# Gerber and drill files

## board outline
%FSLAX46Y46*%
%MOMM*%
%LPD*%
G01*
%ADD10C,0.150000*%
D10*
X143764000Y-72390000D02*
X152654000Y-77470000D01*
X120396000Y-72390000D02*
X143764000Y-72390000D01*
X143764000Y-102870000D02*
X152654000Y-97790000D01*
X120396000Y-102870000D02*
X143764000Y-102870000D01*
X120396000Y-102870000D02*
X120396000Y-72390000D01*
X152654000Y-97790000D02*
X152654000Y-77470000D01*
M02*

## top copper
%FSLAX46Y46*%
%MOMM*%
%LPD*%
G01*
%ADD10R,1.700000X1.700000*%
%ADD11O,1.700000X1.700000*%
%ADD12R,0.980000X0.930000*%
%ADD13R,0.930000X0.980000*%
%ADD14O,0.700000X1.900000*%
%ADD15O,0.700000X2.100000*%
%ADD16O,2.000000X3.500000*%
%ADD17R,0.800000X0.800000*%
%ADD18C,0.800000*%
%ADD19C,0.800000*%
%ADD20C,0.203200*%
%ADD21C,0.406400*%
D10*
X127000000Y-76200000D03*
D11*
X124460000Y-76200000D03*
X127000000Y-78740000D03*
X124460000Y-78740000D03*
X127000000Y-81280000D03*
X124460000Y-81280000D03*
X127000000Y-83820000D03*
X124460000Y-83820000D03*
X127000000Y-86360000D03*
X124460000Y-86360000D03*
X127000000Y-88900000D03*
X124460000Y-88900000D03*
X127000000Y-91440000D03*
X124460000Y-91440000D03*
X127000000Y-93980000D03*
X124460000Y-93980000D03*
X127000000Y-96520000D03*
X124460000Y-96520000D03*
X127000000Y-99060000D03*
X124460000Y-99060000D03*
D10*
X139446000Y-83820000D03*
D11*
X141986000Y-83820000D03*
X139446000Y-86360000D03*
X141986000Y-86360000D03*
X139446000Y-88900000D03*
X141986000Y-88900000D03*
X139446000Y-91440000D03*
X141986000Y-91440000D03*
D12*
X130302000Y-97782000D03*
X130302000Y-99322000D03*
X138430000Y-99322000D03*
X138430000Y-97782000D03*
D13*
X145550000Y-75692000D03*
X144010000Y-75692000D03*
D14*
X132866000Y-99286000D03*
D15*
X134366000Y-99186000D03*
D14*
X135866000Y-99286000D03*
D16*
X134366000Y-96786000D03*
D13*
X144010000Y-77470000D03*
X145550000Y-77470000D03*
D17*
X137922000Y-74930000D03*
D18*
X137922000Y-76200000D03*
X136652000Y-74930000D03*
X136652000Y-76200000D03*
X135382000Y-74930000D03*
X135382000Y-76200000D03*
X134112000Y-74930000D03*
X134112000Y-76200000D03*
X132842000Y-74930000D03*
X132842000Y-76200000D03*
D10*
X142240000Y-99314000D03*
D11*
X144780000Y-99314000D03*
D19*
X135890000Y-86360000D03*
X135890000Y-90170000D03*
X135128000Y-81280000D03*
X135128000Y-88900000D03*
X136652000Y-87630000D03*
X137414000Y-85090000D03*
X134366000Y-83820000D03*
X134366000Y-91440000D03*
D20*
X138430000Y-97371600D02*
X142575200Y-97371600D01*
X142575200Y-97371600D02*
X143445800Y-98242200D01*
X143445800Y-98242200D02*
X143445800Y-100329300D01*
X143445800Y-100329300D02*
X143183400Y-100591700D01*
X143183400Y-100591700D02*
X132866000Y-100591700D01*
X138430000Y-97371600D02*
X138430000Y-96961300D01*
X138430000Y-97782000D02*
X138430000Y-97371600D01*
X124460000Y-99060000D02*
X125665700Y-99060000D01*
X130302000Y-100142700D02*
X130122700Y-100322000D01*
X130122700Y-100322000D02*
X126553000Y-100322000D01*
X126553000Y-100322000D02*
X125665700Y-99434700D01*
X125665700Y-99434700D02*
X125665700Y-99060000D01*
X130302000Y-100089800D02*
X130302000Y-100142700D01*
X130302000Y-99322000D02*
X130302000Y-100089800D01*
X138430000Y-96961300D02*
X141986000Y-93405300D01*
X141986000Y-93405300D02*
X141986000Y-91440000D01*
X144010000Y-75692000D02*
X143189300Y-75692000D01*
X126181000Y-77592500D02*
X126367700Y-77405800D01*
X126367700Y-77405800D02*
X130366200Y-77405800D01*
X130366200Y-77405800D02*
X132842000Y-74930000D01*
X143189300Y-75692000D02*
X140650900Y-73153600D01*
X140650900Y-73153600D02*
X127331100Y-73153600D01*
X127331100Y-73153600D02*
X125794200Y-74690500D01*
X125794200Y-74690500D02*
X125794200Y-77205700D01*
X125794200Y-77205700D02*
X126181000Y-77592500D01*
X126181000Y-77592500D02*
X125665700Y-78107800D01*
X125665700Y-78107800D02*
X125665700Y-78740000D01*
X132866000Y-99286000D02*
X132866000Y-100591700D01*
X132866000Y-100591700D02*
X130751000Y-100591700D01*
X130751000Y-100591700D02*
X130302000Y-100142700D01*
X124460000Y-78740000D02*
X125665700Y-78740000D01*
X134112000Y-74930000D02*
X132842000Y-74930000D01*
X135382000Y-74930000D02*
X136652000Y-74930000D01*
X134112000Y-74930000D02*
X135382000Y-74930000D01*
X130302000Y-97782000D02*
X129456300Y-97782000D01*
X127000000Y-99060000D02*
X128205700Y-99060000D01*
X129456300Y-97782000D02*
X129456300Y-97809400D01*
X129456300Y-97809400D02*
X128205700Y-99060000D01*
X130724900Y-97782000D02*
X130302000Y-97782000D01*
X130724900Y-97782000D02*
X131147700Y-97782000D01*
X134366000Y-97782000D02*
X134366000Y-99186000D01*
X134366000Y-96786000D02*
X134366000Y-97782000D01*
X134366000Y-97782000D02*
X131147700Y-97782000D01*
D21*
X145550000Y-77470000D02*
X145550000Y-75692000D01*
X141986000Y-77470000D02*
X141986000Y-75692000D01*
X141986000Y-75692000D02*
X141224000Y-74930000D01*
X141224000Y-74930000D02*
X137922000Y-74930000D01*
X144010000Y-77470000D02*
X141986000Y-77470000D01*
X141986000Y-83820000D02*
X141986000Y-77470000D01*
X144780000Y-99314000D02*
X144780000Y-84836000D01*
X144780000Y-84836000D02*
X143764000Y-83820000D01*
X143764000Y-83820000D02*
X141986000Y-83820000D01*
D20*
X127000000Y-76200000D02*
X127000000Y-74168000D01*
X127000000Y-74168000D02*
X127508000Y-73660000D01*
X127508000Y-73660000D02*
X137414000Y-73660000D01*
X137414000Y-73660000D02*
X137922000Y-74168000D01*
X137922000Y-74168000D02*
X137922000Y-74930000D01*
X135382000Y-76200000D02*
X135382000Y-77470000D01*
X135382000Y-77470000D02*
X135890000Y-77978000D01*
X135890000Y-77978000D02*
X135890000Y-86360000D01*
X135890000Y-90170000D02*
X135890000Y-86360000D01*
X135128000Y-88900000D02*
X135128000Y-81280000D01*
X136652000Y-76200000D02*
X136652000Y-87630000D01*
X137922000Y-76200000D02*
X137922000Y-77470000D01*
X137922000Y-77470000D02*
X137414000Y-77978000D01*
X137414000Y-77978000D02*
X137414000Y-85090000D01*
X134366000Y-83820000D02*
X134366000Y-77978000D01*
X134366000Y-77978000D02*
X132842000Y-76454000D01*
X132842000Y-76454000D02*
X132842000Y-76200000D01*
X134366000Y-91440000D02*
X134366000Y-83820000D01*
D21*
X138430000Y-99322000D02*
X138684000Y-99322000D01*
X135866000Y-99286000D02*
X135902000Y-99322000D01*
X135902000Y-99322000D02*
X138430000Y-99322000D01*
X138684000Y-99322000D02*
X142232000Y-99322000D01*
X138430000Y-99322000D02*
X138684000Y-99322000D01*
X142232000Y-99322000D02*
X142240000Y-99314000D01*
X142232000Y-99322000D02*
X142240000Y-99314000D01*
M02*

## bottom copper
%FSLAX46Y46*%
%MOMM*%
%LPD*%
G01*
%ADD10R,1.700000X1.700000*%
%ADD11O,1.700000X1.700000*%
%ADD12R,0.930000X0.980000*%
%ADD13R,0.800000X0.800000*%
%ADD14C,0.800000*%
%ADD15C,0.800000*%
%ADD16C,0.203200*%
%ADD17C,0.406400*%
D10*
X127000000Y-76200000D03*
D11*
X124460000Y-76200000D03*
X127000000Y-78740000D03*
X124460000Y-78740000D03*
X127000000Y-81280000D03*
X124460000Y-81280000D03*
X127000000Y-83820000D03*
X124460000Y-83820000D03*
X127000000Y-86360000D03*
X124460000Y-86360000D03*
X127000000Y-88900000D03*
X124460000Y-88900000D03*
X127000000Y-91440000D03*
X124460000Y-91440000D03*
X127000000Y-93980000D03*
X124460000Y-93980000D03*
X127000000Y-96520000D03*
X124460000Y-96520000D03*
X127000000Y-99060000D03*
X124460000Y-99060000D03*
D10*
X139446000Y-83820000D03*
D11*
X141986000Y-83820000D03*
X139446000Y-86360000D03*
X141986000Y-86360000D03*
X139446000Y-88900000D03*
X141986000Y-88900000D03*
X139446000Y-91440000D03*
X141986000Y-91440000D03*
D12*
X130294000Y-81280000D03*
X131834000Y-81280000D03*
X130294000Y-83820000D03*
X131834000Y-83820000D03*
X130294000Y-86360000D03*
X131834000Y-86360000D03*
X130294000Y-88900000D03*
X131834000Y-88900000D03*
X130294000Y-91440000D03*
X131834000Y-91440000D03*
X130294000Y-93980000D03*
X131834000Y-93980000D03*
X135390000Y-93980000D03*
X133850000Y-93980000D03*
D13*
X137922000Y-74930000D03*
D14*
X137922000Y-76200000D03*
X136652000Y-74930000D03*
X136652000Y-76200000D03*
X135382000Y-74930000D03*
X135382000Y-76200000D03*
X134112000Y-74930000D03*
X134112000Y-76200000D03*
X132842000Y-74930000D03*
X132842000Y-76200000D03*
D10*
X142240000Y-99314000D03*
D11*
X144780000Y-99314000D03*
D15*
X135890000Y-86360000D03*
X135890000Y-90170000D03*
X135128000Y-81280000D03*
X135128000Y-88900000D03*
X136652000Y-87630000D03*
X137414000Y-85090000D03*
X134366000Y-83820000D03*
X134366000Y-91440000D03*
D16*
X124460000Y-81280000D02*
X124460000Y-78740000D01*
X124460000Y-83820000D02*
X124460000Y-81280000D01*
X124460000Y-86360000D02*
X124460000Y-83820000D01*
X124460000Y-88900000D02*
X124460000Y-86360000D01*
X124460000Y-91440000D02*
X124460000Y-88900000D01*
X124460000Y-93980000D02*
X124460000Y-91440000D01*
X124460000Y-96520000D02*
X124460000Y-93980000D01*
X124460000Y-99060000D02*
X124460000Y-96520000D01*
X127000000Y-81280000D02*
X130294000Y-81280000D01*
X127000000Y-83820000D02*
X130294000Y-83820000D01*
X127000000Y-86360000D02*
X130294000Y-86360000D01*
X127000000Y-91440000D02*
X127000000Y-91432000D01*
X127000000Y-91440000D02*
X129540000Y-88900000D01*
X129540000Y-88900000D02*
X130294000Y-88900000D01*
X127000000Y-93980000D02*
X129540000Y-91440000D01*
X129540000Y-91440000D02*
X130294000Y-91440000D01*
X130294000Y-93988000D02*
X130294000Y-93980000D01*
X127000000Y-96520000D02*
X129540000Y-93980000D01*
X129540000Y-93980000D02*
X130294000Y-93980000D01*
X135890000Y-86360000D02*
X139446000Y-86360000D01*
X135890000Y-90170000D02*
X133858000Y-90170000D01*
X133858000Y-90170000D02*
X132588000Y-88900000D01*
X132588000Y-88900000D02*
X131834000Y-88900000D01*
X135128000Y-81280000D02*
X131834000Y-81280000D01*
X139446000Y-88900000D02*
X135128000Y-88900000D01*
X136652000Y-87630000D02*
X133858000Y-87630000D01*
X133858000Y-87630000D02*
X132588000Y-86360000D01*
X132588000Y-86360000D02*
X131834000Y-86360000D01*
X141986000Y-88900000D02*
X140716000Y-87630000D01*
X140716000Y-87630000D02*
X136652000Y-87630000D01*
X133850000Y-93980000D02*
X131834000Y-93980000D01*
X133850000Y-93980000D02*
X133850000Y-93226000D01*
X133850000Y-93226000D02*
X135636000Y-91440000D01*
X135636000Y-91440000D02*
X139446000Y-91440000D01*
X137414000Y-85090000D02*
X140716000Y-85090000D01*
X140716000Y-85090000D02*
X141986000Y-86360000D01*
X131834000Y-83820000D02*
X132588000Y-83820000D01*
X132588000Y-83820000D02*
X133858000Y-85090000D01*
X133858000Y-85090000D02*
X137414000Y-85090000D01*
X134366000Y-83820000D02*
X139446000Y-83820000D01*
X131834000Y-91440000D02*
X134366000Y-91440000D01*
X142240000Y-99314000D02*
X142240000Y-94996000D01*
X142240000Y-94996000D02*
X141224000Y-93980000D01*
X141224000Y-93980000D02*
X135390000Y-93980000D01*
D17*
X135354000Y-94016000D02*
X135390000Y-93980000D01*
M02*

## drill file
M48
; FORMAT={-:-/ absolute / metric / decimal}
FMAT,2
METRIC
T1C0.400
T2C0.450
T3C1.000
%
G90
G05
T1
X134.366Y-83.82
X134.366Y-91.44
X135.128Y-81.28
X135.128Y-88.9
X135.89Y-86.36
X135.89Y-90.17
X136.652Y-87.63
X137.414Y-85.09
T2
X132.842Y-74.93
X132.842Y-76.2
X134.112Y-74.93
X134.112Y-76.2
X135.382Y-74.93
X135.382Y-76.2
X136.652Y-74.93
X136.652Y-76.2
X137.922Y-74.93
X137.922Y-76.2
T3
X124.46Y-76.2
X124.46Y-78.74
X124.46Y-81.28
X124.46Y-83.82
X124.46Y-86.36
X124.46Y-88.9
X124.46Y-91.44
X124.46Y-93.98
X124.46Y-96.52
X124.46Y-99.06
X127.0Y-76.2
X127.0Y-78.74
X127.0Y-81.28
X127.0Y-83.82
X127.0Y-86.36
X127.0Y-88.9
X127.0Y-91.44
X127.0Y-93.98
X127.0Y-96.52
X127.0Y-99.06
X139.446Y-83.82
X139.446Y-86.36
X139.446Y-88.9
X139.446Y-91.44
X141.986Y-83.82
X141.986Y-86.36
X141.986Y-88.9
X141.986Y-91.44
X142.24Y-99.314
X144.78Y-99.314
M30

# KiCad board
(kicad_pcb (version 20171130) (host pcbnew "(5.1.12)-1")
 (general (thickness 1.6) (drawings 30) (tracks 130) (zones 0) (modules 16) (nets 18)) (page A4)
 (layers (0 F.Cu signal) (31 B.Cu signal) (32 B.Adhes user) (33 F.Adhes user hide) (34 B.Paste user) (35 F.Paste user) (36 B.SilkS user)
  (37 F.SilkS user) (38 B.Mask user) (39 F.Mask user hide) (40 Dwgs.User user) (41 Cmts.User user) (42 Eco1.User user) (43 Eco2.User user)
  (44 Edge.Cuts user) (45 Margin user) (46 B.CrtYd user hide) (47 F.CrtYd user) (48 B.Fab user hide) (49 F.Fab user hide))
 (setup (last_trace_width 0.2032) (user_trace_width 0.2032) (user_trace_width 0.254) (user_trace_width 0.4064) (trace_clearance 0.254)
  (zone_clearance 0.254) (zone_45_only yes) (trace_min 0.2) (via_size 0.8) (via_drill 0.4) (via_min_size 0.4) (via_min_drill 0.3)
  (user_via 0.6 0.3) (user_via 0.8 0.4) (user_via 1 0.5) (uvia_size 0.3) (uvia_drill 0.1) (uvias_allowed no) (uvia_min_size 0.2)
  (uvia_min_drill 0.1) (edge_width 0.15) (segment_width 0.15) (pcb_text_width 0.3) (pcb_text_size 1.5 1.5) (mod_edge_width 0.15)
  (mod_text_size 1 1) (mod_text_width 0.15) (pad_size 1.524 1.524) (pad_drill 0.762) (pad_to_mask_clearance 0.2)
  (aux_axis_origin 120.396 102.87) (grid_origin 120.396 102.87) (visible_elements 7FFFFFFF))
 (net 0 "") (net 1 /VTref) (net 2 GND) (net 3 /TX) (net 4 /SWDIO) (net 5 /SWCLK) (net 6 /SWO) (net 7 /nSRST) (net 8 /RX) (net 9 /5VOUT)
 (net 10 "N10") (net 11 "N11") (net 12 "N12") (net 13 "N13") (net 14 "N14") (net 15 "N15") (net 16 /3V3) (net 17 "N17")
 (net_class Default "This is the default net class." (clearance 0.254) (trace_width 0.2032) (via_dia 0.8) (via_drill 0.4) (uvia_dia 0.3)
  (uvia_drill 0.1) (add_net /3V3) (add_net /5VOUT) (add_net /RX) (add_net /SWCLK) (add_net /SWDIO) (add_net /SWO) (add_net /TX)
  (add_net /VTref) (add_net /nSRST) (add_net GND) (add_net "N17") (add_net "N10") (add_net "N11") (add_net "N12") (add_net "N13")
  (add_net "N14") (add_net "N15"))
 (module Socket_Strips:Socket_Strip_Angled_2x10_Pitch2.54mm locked (layer F.Cu) (at 127 76.2)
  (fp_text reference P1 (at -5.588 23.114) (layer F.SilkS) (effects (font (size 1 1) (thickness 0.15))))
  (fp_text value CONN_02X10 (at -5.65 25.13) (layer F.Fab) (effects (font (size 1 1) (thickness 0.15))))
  (pad 1 thru_hole rect (at 0 0) (size 1.7 1.7) (drill 1) (layers *.Cu *.Mask) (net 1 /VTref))
  (pad 2 thru_hole oval (at -2.54 0) (size 1.7 1.7) (drill 1) (layers *.Cu *.Mask))
  (pad 3 thru_hole oval (at 0 2.54) (size 1.7 1.7) (drill 1) (layers *.Cu *.Mask))
  (pad 4 thru_hole oval (at -2.54 2.54) (size 1.7 1.7) (drill 1) (layers *.Cu *.Mask) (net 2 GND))
  (pad 5 thru_hole oval (at 0 5.08) (size 1.7 1.7) (drill 1) (layers *.Cu *.Mask) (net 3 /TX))
  (pad 6 thru_hole oval (at -2.54 5.08) (size 1.7 1.7) (drill 1) (layers *.Cu *.Mask) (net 2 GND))
  (pad 7 thru_hole oval (at 0 7.62) (size 1.7 1.7) (drill 1) (layers *.Cu *.Mask) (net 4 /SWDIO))
  (pad 8 thru_hole oval (at -2.54 7.62) (size 1.7 1.7) (drill 1) (layers *.Cu *.Mask) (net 2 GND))
  (pad 9 thru_hole oval (at 0 10.16) (size 1.7 1.7) (drill 1) (layers *.Cu *.Mask) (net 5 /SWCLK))
  (pad 10 thru_hole oval (at -2.54 10.16) (size 1.7 1.7) (drill 1) (layers *.Cu *.Mask) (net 2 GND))
  (pad 11 thru_hole oval (at 0 12.7) (size 1.7 1.7) (drill 1) (layers *.Cu *.Mask))
  (pad 12 thru_hole oval (at -2.54 12.7) (size 1.7 1.7) (drill 1) (layers *.Cu *.Mask) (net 2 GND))
  (pad 13 thru_hole oval (at 0 15.24) (size 1.7 1.7) (drill 1) (layers *.Cu *.Mask) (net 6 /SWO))
  (pad 14 thru_hole oval (at -2.54 15.24) (size 1.7 1.7) (drill 1) (layers *.Cu *.Mask) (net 2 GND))
  (pad 15 thru_hole oval (at 0 17.78) (size 1.7 1.7) (drill 1) (layers *.Cu *.Mask) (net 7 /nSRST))
  (pad 16 thru_hole oval (at -2.54 17.78) (size 1.7 1.7) (drill 1) (layers *.Cu *.Mask) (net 2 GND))
  (pad 17 thru_hole oval (at 0 20.32) (size 1.7 1.7) (drill 1) (layers *.Cu *.Mask) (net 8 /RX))
  (pad 18 thru_hole oval (at -2.54 20.32) (size 1.7 1.7) (drill 1) (layers *.Cu *.Mask) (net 2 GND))
  (pad 19 thru_hole oval (at 0 22.86) (size 1.7 1.7) (drill 1) (layers *.Cu *.Mask) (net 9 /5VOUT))
  (pad 20 thru_hole oval (at -2.54 22.86) (size 1.7 1.7) (drill 1) (layers *.Cu *.Mask) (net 2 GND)))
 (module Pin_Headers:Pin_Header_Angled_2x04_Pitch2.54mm (layer F.Cu) (at 139.446 83.82)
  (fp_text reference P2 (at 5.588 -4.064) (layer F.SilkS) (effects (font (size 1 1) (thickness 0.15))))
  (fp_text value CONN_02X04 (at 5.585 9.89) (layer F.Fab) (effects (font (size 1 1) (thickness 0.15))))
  (pad 1 thru_hole rect (at 0 0) (size 1.7 1.7) (drill 1) (layers *.Cu *.Mask) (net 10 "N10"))
  (pad 2 thru_hole oval (at 2.54 0) (size 1.7 1.7) (drill 1) (layers *.Cu *.Mask) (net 1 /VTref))
  (pad 3 thru_hole oval (at 0 2.54) (size 1.7 1.7) (drill 1) (layers *.Cu *.Mask) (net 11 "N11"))
  (pad 4 thru_hole oval (at 2.54 2.54) (size 1.7 1.7) (drill 1) (layers *.Cu *.Mask) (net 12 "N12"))
  (pad 5 thru_hole oval (at 0 5.08) (size 1.7 1.7) (drill 1) (layers *.Cu *.Mask) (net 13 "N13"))
  (pad 6 thru_hole oval (at 2.54 5.08) (size 1.7 1.7) (drill 1) (layers *.Cu *.Mask) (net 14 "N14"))
  (pad 7 thru_hole oval (at 0 7.62) (size 1.7 1.7) (drill 1) (layers *.Cu *.Mask) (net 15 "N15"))
  (pad 8 thru_hole oval (at 2.54 7.62) (size 1.7 1.7) (drill 1) (layers *.Cu *.Mask) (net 2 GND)))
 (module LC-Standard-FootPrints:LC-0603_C (layer F.Cu) (at 130.302 98.552 270)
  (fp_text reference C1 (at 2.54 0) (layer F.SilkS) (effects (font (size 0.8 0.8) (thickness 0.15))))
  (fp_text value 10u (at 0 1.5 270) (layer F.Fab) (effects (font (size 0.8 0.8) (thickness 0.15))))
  (pad 1 smd rect (at -0.77 0 270) (size 0.93 0.98) (layers F.Cu F.Paste F.Mask) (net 9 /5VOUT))
  (pad 2 smd rect (at 0.77 0 270) (size 0.93 0.98) (layers F.Cu F.Paste F.Mask) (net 2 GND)))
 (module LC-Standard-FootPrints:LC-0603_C (layer F.Cu) (at 138.43 98.552 90)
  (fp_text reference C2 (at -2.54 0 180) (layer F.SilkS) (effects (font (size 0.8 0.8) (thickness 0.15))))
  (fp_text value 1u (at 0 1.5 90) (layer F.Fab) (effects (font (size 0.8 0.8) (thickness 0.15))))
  (pad 1 smd rect (at -0.77 0 90) (size 0.93 0.98) (layers F.Cu F.Paste F.Mask) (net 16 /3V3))
  (pad 2 smd rect (at 0.77 0 90) (size 0.93 0.98) (layers F.Cu F.Paste F.Mask) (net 2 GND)))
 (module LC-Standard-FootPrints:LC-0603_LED (layer F.Cu) (at 144.78 75.692)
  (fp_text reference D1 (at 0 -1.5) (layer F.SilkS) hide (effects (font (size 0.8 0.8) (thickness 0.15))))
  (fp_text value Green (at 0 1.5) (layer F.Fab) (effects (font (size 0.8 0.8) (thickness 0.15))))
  (pad 2 smd rect (at 0.77 0) (size 0.93 0.98) (layers F.Cu F.Paste F.Mask) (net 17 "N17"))
  (pad 1 smd rect (at -0.77 0) (size 0.93 0.98) (layers F.Cu F.Paste F.Mask) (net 2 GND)))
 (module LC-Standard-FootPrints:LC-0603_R (layer B.Cu) (at 131.064 81.28)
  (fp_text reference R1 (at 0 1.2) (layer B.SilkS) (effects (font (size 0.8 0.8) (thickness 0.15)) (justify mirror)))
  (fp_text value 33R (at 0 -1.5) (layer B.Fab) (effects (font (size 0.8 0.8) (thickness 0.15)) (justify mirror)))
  (pad 1 smd rect (at -0.77 0) (size 0.93 0.98) (layers B.Cu B.Paste B.Mask) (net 3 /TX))
  (pad 2 smd rect (at 0.77 0) (size 0.93 0.98) (layers B.Cu B.Paste B.Mask) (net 13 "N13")))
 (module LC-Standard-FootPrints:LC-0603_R (layer B.Cu) (at 131.064 83.82)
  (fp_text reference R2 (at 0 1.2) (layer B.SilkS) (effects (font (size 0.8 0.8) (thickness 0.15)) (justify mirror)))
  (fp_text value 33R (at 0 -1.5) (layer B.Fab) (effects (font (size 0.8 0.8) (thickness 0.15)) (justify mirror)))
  (pad 1 smd rect (at -0.77 0) (size 0.93 0.98) (layers B.Cu B.Paste B.Mask) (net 4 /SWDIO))
  (pad 2 smd rect (at 0.77 0) (size 0.93 0.98) (layers B.Cu B.Paste B.Mask) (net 12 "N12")))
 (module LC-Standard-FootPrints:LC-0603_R (layer B.Cu) (at 131.064 86.36)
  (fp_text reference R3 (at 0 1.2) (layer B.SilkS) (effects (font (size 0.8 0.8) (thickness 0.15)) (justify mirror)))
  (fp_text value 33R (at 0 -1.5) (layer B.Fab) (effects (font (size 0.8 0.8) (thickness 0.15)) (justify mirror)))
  (pad 1 smd rect (at -0.77 0) (size 0.93 0.98) (layers B.Cu B.Paste B.Mask) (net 5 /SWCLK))
  (pad 2 smd rect (at 0.77 0) (size 0.93 0.98) (layers B.Cu B.Paste B.Mask) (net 14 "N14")))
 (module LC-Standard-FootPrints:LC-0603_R (layer B.Cu) (at 131.064 88.9)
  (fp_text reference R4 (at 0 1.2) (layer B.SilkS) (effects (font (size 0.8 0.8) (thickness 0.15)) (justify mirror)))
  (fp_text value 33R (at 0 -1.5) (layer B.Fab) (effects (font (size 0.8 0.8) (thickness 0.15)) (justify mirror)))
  (pad 1 smd rect (at -0.77 0) (size 0.93 0.98) (layers B.Cu B.Paste B.Mask) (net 6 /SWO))
  (pad 2 smd rect (at 0.77 0) (size 0.93 0.98) (layers B.Cu B.Paste B.Mask) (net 11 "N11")))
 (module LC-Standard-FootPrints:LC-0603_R (layer B.Cu) (at 131.064 91.44)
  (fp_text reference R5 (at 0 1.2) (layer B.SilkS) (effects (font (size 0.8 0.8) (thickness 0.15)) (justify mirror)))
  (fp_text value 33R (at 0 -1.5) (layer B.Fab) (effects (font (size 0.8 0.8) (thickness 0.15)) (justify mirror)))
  (pad 1 smd rect (at -0.77 0) (size 0.93 0.98) (layers B.Cu B.Paste B.Mask) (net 7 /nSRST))
  (pad 2 smd rect (at 0.77 0) (size 0.93 0.98) (layers B.Cu B.Paste B.Mask) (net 10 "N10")))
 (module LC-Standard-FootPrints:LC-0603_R (layer B.Cu) (at 131.064 93.98)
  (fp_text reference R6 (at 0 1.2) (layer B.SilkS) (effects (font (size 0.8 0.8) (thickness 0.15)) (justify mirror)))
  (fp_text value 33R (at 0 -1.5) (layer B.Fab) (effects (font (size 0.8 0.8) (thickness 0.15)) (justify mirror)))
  (pad 1 smd rect (at -0.77 0) (size 0.93 0.98) (layers B.Cu B.Paste B.Mask) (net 8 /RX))
  (pad 2 smd rect (at 0.77 0) (size 0.93 0.98) (layers B.Cu B.Paste B.Mask) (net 15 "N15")))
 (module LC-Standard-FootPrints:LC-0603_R (layer B.Cu) (at 134.62 93.98 180)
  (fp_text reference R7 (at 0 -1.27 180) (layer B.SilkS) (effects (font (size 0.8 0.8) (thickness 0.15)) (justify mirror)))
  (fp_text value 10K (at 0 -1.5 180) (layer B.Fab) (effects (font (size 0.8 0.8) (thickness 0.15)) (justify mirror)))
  (pad 1 smd rect (at -0.77 0 180) (size 0.93 0.98) (layers B.Cu B.Paste B.Mask) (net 16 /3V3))
  (pad 2 smd rect (at 0.77 0 180) (size 0.93 0.98) (layers B.Cu B.Paste B.Mask) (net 15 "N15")))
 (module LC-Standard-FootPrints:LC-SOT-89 (layer F.Cu) (at 134.366 97.536 270)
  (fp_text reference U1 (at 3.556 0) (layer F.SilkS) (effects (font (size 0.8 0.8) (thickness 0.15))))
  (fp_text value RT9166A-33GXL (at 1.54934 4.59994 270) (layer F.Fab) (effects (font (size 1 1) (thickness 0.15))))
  (pad 1 smd oval (at 1.75 1.5) (size 0.7 1.9) (layers F.Cu F.Paste F.Mask) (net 2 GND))
  (pad 2 smd oval (at 1.65 0) (size 0.7 2.1) (layers F.Cu F.Paste F.Mask) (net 9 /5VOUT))
  (pad 3 smd oval (at 1.75 -1.5) (size 0.7 1.9) (layers F.Cu F.Paste F.Mask) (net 16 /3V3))
  (pad 2 smd oval (at -0.75 0) (size 2 3.5) (layers F.Cu F.Paste F.Mask) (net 9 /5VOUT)))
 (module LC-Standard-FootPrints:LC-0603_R (layer F.Cu) (at 144.78 77.47)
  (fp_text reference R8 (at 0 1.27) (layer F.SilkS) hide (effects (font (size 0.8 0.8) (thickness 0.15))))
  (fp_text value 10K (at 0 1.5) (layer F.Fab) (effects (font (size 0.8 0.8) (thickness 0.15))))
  (pad 1 smd rect (at -0.77 0) (size 0.93 0.98) (layers F.Cu F.Paste F.Mask) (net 1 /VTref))
  (pad 2 smd rect (at 0.77 0) (size 0.93 0.98) (layers F.Cu F.Paste F.Mask) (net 17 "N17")))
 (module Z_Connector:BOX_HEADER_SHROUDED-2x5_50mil (layer F.Cu) (at 137.922 74.93 180)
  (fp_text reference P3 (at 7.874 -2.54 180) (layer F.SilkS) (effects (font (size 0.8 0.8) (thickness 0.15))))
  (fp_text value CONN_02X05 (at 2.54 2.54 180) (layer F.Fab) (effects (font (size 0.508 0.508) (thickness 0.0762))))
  (pad 1 thru_hole rect (at 0 0 180) (size 0.8 0.8) (drill 0.45) (layers *.Cu *.Mask) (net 1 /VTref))
  (pad 2 thru_hole circle (at 0 -1.27 180) (size 0.8 0.8) (drill 0.45) (layers *.Cu *.Mask) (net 12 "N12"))
  (pad 3 thru_hole circle (at 1.27 0 180) (size 0.8 0.8) (drill 0.45) (layers *.Cu *.Mask) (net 2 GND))
  (pad 4 thru_hole circle (at 1.27 -1.27 180) (size 0.8 0.8) (drill 0.45) (layers *.Cu *.Mask) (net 14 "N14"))
  (pad 5 thru_hole circle (at 2.54 0 180) (size 0.8 0.8) (drill 0.45) (layers *.Cu *.Mask) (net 2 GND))
  (pad 6 thru_hole circle (at 2.54 -1.27 180) (size 0.8 0.8) (drill 0.45) (layers *.Cu *.Mask) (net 11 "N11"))
  (pad 7 thru_hole circle (at 3.81 0 180) (size 0.8 0.8) (drill 0.45) (layers *.Cu *.Mask) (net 2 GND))
  (pad 8 thru_hole circle (at 3.81 -1.27 180) (size 0.8 0.8) (drill 0.45) (layers *.Cu *.Mask))
  (pad 9 thru_hole circle (at 5.08 0 180) (size 0.8 0.8) (drill 0.45) (layers *.Cu *.Mask) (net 2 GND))
  (pad 10 thru_hole circle (at 5.08 -1.27 180) (size 0.8 0.8) (drill 0.45) (layers *.Cu *.Mask) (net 10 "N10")))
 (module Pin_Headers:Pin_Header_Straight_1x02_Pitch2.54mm (layer F.Cu) (at 142.24 99.314 90)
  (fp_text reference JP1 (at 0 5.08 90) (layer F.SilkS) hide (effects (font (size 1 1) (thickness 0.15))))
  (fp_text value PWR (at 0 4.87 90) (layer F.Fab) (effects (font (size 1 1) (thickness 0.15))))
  (pad 1 thru_hole rect (at 0 0 90) (size 1.7 1.7) (drill 1) (layers *.Cu *.Mask) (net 16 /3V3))
  (pad 2 thru_hole oval (at 0 2.54 90) (size 1.7 1.7) (drill 1) (layers *.Cu *.Mask) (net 1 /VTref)))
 (gr_line (start 143.764 72.39) (end 152.654 77.47) (angle 90) (layer Edge.Cuts) (width 0.15))
 (gr_line (start 120.396 72.39) (end 143.764 72.39) (angle 90) (layer Edge.Cuts) (width 0.15))
 (gr_line (start 143.764 102.87) (end 152.654 97.79) (angle 90) (layer Edge.Cuts) (width 0.15))
 (gr_line (start 120.396 102.87) (end 143.764 102.87) (angle 90) (layer Edge.Cuts) (width 0.15))
 (gr_line (start 120.396 102.87) (end 120.396 72.39) (angle 90) (layer Edge.Cuts) (width 0.15))
 (gr_line (start 152.654 97.79) (end 152.654 77.47) (angle 90) (layer Edge.Cuts) (width 0.15))
 (segment (start 124.46 81.28) (end 124.46 78.74) (width 0.2032) (layer B.Cu) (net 2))
 (segment (start 124.46 83.82) (end 124.46 81.28) (width 0.2032) (layer B.Cu) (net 2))
 (segment (start 124.46 86.36) (end 124.46 83.82) (width 0.2032) (layer B.Cu) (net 2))
 (segment (start 124.46 88.9) (end 124.46 86.36) (width 0.2032) (layer B.Cu) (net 2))
 (segment (start 124.46 91.44) (end 124.46 88.9) (width 0.2032) (layer B.Cu) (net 2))
 (segment (start 124.46 93.98) (end 124.46 91.44) (width 0.2032) (layer B.Cu) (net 2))
 (segment (start 124.46 96.52) (end 124.46 93.98) (width 0.2032) (layer B.Cu) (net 2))
 (segment (start 124.46 99.06) (end 124.46 96.52) (width 0.2032) (layer B.Cu) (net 2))
 (segment (start 138.43 97.3716) (end 142.5752 97.3716) (width 0.2032) (layer F.Cu) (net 2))
 (segment (start 142.5752 97.3716) (end 143.4458 98.2422) (width 0.2032) (layer F.Cu) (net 2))
 (segment (start 143.4458 98.2422) (end 143.4458 100.3293) (width 0.2032) (layer F.Cu) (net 2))
 (segment (start 143.4458 100.3293) (end 143.1834 100.5917) (width 0.2032) (layer F.Cu) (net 2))
 (segment (start 143.1834 100.5917) (end 132.866 100.5917) (width 0.2032) (layer F.Cu) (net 2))
 (segment (start 138.43 97.3716) (end 138.43 96.9613) (width 0.2032) (layer F.Cu) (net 2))
 (segment (start 138.43 97.782) (end 138.43 97.3716) (width 0.2032) (layer F.Cu) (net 2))
 (segment (start 124.46 99.06) (end 125.6657 99.06) (width 0.2032) (layer F.Cu) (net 2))
 (segment (start 130.302 100.1427) (end 130.1227 100.322) (width 0.2032) (layer F.Cu) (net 2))
 (segment (start 130.1227 100.322) (end 126.553 100.322) (width 0.2032) (layer F.Cu) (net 2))
 (segment (start 126.553 100.322) (end 125.6657 99.4347) (width 0.2032) (layer F.Cu) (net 2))
 (segment (start 125.6657 99.4347) (end 125.6657 99.06) (width 0.2032) (layer F.Cu) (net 2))
 (segment (start 130.302 100.0898) (end 130.302 100.1427) (width 0.2032) (layer F.Cu) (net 2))
 (segment (start 130.302 99.322) (end 130.302 100.0898) (width 0.2032) (layer F.Cu) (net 2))
 (segment (start 138.43 96.9613) (end 141.986 93.4053) (width 0.2032) (layer F.Cu) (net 2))
 (segment (start 141.986 93.4053) (end 141.986 91.44) (width 0.2032) (layer F.Cu) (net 2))
 (segment (start 144.01 75.692) (end 143.1893 75.692) (width 0.2032) (layer F.Cu) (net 2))
 (segment (start 126.181 77.5925) (end 126.3677 77.4058) (width 0.2032) (layer F.Cu) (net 2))
 (segment (start 126.3677 77.4058) (end 130.3662 77.4058) (width 0.2032) (layer F.Cu) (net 2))
 (segment (start 130.3662 77.4058) (end 132.842 74.93) (width 0.2032) (layer F.Cu) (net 2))
 (segment (start 143.1893 75.692) (end 140.6509 73.1536) (width 0.2032) (layer F.Cu) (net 2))
 (segment (start 140.6509 73.1536) (end 127.3311 73.1536) (width 0.2032) (layer F.Cu) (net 2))
 (segment (start 127.3311 73.1536) (end 125.7942 74.6905) (width 0.2032) (layer F.Cu) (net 2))
 (segment (start 125.7942 74.6905) (end 125.7942 77.2057) (width 0.2032) (layer F.Cu) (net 2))
 (segment (start 125.7942 77.2057) (end 126.181 77.5925) (width 0.2032) (layer F.Cu) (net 2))
 (segment (start 126.181 77.5925) (end 125.6657 78.1078) (width 0.2032) (layer F.Cu) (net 2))
 (segment (start 125.6657 78.1078) (end 125.6657 78.74) (width 0.2032) (layer F.Cu) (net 2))
 (segment (start 132.866 99.286) (end 132.866 100.5917) (width 0.2032) (layer F.Cu) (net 2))
 (segment (start 132.866 100.5917) (end 130.751 100.5917) (width 0.2032) (layer F.Cu) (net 2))
 (segment (start 130.751 100.5917) (end 130.302 100.1427) (width 0.2032) (layer F.Cu) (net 2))
 (segment (start 124.46 78.74) (end 125.6657 78.74) (width 0.2032) (layer F.Cu) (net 2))
 (segment (start 134.112 74.93) (end 132.842 74.93) (width 0.2032) (layer F.Cu) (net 2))
 (segment (start 135.382 74.93) (end 136.652 74.93) (width 0.2032) (layer F.Cu) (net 2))
 (segment (start 134.112 74.93) (end 135.382 74.93) (width 0.2032) (layer F.Cu) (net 2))
 (segment (start 130.302 97.782) (end 129.4563 97.782) (width 0.2032) (layer F.Cu) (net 9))
 (segment (start 127 99.06) (end 128.2057 99.06) (width 0.2032) (layer F.Cu) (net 9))
 (segment (start 129.4563 97.782) (end 129.4563 97.8094) (width 0.2032) (layer F.Cu) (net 9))
 (segment (start 129.4563 97.8094) (end 128.2057 99.06) (width 0.2032) (layer F.Cu) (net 9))
 (segment (start 130.7249 97.782) (end 130.302 97.782) (width 0.2032) (layer F.Cu) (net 9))
 (segment (start 130.7249 97.782) (end 131.1477 97.782) (width 0.2032) (layer F.Cu) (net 9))
 (segment (start 134.366 97.782) (end 134.366 99.186) (width 0.2032) (layer F.Cu) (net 9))
 (segment (start 134.366 96.786) (end 134.366 97.782) (width 0.2032) (layer F.Cu) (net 9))
 (segment (start 134.366 97.782) (end 131.1477 97.782) (width 0.2032) (layer F.Cu) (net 9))
 (segment (start 145.55 77.47) (end 145.55 75.692) (width 0.4064) (layer F.Cu) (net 17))
 (segment (start 141.986 77.47) (end 141.986 75.692) (width 0.4064) (layer F.Cu) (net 1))
 (segment (start 141.986 75.692) (end 141.224 74.93) (width 0.4064) (layer F.Cu) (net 1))
 (segment (start 141.224 74.93) (end 137.922 74.93) (width 0.4064) (layer F.Cu) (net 1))
 (segment (start 144.01 77.47) (end 141.986 77.47) (width 0.4064) (layer F.Cu) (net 1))
 (segment (start 141.986 83.82) (end 141.986 77.47) (width 0.4064) (layer F.Cu) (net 1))
 (segment (start 144.78 99.314) (end 144.78 84.836) (width 0.4064) (layer F.Cu) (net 1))
 (segment (start 144.78 84.836) (end 143.764 83.82) (width 0.4064) (layer F.Cu) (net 1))
 (segment (start 143.764 83.82) (end 141.986 83.82) (width 0.4064) (layer F.Cu) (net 1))
 (segment (start 127 76.2) (end 127 74.168) (width 0.2032) (layer F.Cu) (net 1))
 (segment (start 127 74.168) (end 127.508 73.66) (width 0.2032) (layer F.Cu) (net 1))
 (segment (start 127.508 73.66) (end 137.414 73.66) (width 0.2032) (layer F.Cu) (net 1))
 (segment (start 137.414 73.66) (end 137.922 74.168) (width 0.2032) (layer F.Cu) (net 1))
 (segment (start 137.922 74.168) (end 137.922 74.93) (width 0.2032) (layer F.Cu) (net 1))
 (segment (start 127 81.28) (end 130.294 81.28) (width 0.2032) (layer B.Cu) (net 3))
 (segment (start 127 83.82) (end 130.294 83.82) (width 0.2032) (layer B.Cu) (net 4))
 (segment (start 127 86.36) (end 130.294 86.36) (width 0.2032) (layer B.Cu) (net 5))
 (segment (start 127 91.44) (end 127 91.432) (width 0.2032) (layer B.Cu) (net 6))
 (segment (start 127 91.44) (end 129.54 88.9) (width 0.2032) (layer B.Cu) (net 6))
 (segment (start 129.54 88.9) (end 130.294 88.9) (width 0.2032) (layer B.Cu) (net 6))
 (segment (start 127 93.98) (end 129.54 91.44) (width 0.2032) (layer B.Cu) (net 7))
 (segment (start 129.54 91.44) (end 130.294 91.44) (width 0.2032) (layer B.Cu) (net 7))
 (segment (start 130.294 93.988) (end 130.294 93.98) (width 0.2032) (layer B.Cu) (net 8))
 (segment (start 127 96.52) (end 129.54 93.98) (width 0.2032) (layer B.Cu) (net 8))
 (segment (start 129.54 93.98) (end 130.294 93.98) (width 0.2032) (layer B.Cu) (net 8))
 (segment (start 135.382 76.2) (end 135.382 77.47) (width 0.2032) (layer F.Cu) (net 11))
 (segment (start 135.382 77.47) (end 135.89 77.978) (width 0.2032) (layer F.Cu) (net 11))
 (segment (start 135.89 77.978) (end 135.89 86.36) (width 0.2032) (layer F.Cu) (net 11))
 (segment (start 135.89 86.36) (end 139.446 86.36) (width 0.2032) (layer B.Cu) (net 11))
 (segment (start 135.89 90.17) (end 133.858 90.17) (width 0.2032) (layer B.Cu) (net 11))
 (segment (start 133.858 90.17) (end 132.588 88.9) (width 0.2032) (layer B.Cu) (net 11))
 (segment (start 132.588 88.9) (end 131.834 88.9) (width 0.2032) (layer B.Cu) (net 11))
 (segment (start 135.89 90.17) (end 135.89 86.36) (width 0.2032) (layer F.Cu) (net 11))
 (via (at 135.89 86.36) (size 0.8) (layers F.Cu B.Cu) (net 11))
 (via (at 135.89 90.17) (size 0.8) (layers F.Cu B.Cu) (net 11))
 (segment (start 135.128 81.28) (end 131.834 81.28) (width 0.2032) (layer B.Cu) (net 13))
 (segment (start 135.128 88.9) (end 135.128 81.28) (width 0.2032) (layer F.Cu) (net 13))
 (segment (start 139.446 88.9) (end 135.128 88.9) (width 0.2032) (layer B.Cu) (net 13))
 (via (at 135.128 81.28) (size 0.8) (layers F.Cu B.Cu) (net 13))
 (via (at 135.128 88.9) (size 0.8) (layers F.Cu B.Cu) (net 13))
 (segment (start 136.652 87.63) (end 133.858 87.63) (width 0.2032) (layer B.Cu) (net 14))
 (segment (start 133.858 87.63) (end 132.588 86.36) (width 0.2032) (layer B.Cu) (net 14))
 (segment (start 132.588 86.36) (end 131.834 86.36) (width 0.2032) (layer B.Cu) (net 14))
 (segment (start 141.986 88.9) (end 140.716 87.63) (width 0.2032) (layer B.Cu) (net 14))
 (segment (start 140.716 87.63) (end 136.652 87.63) (width 0.2032) (layer B.Cu) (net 14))
 (segment (start 136.652 76.2) (end 136.652 87.63) (width 0.2032) (layer F.Cu) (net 14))
 (via (at 136.652 87.63) (size 0.8) (layers F.Cu B.Cu) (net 14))
 (segment (start 133.85 93.98) (end 131.834 93.98) (width 0.2032) (layer B.Cu) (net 15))
 (segment (start 133.85 93.98) (end 133.85 93.226) (width 0.2032) (layer B.Cu) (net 15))
 (segment (start 133.85 93.226) (end 135.636 91.44) (width 0.2032) (layer B.Cu) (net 15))
 (segment (start 135.636 91.44) (end 139.446 91.44) (width 0.2032) (layer B.Cu) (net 15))
 (segment (start 137.414 85.09) (end 140.716 85.09) (width 0.2032) (layer B.Cu) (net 12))
 (segment (start 140.716 85.09) (end 141.986 86.36) (width 0.2032) (layer B.Cu) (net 12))
 (segment (start 131.834 83.82) (end 132.588 83.82) (width 0.2032) (layer B.Cu) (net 12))
 (segment (start 132.588 83.82) (end 133.858 85.09) (width 0.2032) (layer B.Cu) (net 12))
 (segment (start 133.858 85.09) (end 137.414 85.09) (width 0.2032) (layer B.Cu) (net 12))
 (segment (start 137.922 76.2) (end 137.922 77.47) (width 0.2032) (layer F.Cu) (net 12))
 (segment (start 137.922 77.47) (end 137.414 77.978) (width 0.2032) (layer F.Cu) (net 12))
 (segment (start 137.414 77.978) (end 137.414 85.09) (width 0.2032) (layer F.Cu) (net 12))
 (via (at 137.414 85.09) (size 0.8) (layers F.Cu B.Cu) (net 12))
 (segment (start 134.366 83.82) (end 139.446 83.82) (width 0.2032) (layer B.Cu) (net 10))
 (segment (start 134.366 83.82) (end 134.366 77.978) (width 0.2032) (layer F.Cu) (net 10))
 (segment (start 134.366 77.978) (end 132.842 76.454) (width 0.2032) (layer F.Cu) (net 10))
 (segment (start 132.842 76.454) (end 132.842 76.2) (width 0.2032) (layer F.Cu) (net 10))
 (segment (start 134.366 91.44) (end 134.366 83.82) (width 0.2032) (layer F.Cu) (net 10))
 (segment (start 131.834 91.44) (end 134.366 91.44) (width 0.2032) (layer B.Cu) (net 10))
 (via (at 134.366 83.82) (size 0.8) (layers F.Cu B.Cu) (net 10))
 (via (at 134.366 91.44) (size 0.8) (layers F.Cu B.Cu) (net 10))
 (segment (start 138.43 99.322) (end 138.684 99.322) (width 0.4064) (layer F.Cu) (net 16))
 (segment (start 135.866 99.286) (end 135.902 99.322) (width 0.4064) (layer F.Cu) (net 16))
 (segment (start 135.902 99.322) (end 138.43 99.322) (width 0.4064) (layer F.Cu) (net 16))
 (segment (start 138.684 99.322) (end 142.232 99.322) (width 0.4064) (layer F.Cu) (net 16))
 (segment (start 138.43 99.322) (end 138.684 99.322) (width 0.4064) (layer F.Cu) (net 16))
 (segment (start 142.232 99.322) (end 142.24 99.314) (width 0.4064) (layer F.Cu) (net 16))
 (segment (start 142.232 99.322) (end 142.24 99.314) (width 0.4064) (layer F.Cu) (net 16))
 (segment (start 142.24 99.314) (end 142.24 94.996) (width 0.2032) (layer B.Cu) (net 16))
 (segment (start 142.24 94.996) (end 141.224 93.98) (width 0.2032) (layer B.Cu) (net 16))
 (segment (start 141.224 93.98) (end 135.39 93.98) (width 0.2032) (layer B.Cu) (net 16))
 (segment (start 135.354 94.016) (end 135.39 93.98) (width 0.4064) (layer B.Cu) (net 16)))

